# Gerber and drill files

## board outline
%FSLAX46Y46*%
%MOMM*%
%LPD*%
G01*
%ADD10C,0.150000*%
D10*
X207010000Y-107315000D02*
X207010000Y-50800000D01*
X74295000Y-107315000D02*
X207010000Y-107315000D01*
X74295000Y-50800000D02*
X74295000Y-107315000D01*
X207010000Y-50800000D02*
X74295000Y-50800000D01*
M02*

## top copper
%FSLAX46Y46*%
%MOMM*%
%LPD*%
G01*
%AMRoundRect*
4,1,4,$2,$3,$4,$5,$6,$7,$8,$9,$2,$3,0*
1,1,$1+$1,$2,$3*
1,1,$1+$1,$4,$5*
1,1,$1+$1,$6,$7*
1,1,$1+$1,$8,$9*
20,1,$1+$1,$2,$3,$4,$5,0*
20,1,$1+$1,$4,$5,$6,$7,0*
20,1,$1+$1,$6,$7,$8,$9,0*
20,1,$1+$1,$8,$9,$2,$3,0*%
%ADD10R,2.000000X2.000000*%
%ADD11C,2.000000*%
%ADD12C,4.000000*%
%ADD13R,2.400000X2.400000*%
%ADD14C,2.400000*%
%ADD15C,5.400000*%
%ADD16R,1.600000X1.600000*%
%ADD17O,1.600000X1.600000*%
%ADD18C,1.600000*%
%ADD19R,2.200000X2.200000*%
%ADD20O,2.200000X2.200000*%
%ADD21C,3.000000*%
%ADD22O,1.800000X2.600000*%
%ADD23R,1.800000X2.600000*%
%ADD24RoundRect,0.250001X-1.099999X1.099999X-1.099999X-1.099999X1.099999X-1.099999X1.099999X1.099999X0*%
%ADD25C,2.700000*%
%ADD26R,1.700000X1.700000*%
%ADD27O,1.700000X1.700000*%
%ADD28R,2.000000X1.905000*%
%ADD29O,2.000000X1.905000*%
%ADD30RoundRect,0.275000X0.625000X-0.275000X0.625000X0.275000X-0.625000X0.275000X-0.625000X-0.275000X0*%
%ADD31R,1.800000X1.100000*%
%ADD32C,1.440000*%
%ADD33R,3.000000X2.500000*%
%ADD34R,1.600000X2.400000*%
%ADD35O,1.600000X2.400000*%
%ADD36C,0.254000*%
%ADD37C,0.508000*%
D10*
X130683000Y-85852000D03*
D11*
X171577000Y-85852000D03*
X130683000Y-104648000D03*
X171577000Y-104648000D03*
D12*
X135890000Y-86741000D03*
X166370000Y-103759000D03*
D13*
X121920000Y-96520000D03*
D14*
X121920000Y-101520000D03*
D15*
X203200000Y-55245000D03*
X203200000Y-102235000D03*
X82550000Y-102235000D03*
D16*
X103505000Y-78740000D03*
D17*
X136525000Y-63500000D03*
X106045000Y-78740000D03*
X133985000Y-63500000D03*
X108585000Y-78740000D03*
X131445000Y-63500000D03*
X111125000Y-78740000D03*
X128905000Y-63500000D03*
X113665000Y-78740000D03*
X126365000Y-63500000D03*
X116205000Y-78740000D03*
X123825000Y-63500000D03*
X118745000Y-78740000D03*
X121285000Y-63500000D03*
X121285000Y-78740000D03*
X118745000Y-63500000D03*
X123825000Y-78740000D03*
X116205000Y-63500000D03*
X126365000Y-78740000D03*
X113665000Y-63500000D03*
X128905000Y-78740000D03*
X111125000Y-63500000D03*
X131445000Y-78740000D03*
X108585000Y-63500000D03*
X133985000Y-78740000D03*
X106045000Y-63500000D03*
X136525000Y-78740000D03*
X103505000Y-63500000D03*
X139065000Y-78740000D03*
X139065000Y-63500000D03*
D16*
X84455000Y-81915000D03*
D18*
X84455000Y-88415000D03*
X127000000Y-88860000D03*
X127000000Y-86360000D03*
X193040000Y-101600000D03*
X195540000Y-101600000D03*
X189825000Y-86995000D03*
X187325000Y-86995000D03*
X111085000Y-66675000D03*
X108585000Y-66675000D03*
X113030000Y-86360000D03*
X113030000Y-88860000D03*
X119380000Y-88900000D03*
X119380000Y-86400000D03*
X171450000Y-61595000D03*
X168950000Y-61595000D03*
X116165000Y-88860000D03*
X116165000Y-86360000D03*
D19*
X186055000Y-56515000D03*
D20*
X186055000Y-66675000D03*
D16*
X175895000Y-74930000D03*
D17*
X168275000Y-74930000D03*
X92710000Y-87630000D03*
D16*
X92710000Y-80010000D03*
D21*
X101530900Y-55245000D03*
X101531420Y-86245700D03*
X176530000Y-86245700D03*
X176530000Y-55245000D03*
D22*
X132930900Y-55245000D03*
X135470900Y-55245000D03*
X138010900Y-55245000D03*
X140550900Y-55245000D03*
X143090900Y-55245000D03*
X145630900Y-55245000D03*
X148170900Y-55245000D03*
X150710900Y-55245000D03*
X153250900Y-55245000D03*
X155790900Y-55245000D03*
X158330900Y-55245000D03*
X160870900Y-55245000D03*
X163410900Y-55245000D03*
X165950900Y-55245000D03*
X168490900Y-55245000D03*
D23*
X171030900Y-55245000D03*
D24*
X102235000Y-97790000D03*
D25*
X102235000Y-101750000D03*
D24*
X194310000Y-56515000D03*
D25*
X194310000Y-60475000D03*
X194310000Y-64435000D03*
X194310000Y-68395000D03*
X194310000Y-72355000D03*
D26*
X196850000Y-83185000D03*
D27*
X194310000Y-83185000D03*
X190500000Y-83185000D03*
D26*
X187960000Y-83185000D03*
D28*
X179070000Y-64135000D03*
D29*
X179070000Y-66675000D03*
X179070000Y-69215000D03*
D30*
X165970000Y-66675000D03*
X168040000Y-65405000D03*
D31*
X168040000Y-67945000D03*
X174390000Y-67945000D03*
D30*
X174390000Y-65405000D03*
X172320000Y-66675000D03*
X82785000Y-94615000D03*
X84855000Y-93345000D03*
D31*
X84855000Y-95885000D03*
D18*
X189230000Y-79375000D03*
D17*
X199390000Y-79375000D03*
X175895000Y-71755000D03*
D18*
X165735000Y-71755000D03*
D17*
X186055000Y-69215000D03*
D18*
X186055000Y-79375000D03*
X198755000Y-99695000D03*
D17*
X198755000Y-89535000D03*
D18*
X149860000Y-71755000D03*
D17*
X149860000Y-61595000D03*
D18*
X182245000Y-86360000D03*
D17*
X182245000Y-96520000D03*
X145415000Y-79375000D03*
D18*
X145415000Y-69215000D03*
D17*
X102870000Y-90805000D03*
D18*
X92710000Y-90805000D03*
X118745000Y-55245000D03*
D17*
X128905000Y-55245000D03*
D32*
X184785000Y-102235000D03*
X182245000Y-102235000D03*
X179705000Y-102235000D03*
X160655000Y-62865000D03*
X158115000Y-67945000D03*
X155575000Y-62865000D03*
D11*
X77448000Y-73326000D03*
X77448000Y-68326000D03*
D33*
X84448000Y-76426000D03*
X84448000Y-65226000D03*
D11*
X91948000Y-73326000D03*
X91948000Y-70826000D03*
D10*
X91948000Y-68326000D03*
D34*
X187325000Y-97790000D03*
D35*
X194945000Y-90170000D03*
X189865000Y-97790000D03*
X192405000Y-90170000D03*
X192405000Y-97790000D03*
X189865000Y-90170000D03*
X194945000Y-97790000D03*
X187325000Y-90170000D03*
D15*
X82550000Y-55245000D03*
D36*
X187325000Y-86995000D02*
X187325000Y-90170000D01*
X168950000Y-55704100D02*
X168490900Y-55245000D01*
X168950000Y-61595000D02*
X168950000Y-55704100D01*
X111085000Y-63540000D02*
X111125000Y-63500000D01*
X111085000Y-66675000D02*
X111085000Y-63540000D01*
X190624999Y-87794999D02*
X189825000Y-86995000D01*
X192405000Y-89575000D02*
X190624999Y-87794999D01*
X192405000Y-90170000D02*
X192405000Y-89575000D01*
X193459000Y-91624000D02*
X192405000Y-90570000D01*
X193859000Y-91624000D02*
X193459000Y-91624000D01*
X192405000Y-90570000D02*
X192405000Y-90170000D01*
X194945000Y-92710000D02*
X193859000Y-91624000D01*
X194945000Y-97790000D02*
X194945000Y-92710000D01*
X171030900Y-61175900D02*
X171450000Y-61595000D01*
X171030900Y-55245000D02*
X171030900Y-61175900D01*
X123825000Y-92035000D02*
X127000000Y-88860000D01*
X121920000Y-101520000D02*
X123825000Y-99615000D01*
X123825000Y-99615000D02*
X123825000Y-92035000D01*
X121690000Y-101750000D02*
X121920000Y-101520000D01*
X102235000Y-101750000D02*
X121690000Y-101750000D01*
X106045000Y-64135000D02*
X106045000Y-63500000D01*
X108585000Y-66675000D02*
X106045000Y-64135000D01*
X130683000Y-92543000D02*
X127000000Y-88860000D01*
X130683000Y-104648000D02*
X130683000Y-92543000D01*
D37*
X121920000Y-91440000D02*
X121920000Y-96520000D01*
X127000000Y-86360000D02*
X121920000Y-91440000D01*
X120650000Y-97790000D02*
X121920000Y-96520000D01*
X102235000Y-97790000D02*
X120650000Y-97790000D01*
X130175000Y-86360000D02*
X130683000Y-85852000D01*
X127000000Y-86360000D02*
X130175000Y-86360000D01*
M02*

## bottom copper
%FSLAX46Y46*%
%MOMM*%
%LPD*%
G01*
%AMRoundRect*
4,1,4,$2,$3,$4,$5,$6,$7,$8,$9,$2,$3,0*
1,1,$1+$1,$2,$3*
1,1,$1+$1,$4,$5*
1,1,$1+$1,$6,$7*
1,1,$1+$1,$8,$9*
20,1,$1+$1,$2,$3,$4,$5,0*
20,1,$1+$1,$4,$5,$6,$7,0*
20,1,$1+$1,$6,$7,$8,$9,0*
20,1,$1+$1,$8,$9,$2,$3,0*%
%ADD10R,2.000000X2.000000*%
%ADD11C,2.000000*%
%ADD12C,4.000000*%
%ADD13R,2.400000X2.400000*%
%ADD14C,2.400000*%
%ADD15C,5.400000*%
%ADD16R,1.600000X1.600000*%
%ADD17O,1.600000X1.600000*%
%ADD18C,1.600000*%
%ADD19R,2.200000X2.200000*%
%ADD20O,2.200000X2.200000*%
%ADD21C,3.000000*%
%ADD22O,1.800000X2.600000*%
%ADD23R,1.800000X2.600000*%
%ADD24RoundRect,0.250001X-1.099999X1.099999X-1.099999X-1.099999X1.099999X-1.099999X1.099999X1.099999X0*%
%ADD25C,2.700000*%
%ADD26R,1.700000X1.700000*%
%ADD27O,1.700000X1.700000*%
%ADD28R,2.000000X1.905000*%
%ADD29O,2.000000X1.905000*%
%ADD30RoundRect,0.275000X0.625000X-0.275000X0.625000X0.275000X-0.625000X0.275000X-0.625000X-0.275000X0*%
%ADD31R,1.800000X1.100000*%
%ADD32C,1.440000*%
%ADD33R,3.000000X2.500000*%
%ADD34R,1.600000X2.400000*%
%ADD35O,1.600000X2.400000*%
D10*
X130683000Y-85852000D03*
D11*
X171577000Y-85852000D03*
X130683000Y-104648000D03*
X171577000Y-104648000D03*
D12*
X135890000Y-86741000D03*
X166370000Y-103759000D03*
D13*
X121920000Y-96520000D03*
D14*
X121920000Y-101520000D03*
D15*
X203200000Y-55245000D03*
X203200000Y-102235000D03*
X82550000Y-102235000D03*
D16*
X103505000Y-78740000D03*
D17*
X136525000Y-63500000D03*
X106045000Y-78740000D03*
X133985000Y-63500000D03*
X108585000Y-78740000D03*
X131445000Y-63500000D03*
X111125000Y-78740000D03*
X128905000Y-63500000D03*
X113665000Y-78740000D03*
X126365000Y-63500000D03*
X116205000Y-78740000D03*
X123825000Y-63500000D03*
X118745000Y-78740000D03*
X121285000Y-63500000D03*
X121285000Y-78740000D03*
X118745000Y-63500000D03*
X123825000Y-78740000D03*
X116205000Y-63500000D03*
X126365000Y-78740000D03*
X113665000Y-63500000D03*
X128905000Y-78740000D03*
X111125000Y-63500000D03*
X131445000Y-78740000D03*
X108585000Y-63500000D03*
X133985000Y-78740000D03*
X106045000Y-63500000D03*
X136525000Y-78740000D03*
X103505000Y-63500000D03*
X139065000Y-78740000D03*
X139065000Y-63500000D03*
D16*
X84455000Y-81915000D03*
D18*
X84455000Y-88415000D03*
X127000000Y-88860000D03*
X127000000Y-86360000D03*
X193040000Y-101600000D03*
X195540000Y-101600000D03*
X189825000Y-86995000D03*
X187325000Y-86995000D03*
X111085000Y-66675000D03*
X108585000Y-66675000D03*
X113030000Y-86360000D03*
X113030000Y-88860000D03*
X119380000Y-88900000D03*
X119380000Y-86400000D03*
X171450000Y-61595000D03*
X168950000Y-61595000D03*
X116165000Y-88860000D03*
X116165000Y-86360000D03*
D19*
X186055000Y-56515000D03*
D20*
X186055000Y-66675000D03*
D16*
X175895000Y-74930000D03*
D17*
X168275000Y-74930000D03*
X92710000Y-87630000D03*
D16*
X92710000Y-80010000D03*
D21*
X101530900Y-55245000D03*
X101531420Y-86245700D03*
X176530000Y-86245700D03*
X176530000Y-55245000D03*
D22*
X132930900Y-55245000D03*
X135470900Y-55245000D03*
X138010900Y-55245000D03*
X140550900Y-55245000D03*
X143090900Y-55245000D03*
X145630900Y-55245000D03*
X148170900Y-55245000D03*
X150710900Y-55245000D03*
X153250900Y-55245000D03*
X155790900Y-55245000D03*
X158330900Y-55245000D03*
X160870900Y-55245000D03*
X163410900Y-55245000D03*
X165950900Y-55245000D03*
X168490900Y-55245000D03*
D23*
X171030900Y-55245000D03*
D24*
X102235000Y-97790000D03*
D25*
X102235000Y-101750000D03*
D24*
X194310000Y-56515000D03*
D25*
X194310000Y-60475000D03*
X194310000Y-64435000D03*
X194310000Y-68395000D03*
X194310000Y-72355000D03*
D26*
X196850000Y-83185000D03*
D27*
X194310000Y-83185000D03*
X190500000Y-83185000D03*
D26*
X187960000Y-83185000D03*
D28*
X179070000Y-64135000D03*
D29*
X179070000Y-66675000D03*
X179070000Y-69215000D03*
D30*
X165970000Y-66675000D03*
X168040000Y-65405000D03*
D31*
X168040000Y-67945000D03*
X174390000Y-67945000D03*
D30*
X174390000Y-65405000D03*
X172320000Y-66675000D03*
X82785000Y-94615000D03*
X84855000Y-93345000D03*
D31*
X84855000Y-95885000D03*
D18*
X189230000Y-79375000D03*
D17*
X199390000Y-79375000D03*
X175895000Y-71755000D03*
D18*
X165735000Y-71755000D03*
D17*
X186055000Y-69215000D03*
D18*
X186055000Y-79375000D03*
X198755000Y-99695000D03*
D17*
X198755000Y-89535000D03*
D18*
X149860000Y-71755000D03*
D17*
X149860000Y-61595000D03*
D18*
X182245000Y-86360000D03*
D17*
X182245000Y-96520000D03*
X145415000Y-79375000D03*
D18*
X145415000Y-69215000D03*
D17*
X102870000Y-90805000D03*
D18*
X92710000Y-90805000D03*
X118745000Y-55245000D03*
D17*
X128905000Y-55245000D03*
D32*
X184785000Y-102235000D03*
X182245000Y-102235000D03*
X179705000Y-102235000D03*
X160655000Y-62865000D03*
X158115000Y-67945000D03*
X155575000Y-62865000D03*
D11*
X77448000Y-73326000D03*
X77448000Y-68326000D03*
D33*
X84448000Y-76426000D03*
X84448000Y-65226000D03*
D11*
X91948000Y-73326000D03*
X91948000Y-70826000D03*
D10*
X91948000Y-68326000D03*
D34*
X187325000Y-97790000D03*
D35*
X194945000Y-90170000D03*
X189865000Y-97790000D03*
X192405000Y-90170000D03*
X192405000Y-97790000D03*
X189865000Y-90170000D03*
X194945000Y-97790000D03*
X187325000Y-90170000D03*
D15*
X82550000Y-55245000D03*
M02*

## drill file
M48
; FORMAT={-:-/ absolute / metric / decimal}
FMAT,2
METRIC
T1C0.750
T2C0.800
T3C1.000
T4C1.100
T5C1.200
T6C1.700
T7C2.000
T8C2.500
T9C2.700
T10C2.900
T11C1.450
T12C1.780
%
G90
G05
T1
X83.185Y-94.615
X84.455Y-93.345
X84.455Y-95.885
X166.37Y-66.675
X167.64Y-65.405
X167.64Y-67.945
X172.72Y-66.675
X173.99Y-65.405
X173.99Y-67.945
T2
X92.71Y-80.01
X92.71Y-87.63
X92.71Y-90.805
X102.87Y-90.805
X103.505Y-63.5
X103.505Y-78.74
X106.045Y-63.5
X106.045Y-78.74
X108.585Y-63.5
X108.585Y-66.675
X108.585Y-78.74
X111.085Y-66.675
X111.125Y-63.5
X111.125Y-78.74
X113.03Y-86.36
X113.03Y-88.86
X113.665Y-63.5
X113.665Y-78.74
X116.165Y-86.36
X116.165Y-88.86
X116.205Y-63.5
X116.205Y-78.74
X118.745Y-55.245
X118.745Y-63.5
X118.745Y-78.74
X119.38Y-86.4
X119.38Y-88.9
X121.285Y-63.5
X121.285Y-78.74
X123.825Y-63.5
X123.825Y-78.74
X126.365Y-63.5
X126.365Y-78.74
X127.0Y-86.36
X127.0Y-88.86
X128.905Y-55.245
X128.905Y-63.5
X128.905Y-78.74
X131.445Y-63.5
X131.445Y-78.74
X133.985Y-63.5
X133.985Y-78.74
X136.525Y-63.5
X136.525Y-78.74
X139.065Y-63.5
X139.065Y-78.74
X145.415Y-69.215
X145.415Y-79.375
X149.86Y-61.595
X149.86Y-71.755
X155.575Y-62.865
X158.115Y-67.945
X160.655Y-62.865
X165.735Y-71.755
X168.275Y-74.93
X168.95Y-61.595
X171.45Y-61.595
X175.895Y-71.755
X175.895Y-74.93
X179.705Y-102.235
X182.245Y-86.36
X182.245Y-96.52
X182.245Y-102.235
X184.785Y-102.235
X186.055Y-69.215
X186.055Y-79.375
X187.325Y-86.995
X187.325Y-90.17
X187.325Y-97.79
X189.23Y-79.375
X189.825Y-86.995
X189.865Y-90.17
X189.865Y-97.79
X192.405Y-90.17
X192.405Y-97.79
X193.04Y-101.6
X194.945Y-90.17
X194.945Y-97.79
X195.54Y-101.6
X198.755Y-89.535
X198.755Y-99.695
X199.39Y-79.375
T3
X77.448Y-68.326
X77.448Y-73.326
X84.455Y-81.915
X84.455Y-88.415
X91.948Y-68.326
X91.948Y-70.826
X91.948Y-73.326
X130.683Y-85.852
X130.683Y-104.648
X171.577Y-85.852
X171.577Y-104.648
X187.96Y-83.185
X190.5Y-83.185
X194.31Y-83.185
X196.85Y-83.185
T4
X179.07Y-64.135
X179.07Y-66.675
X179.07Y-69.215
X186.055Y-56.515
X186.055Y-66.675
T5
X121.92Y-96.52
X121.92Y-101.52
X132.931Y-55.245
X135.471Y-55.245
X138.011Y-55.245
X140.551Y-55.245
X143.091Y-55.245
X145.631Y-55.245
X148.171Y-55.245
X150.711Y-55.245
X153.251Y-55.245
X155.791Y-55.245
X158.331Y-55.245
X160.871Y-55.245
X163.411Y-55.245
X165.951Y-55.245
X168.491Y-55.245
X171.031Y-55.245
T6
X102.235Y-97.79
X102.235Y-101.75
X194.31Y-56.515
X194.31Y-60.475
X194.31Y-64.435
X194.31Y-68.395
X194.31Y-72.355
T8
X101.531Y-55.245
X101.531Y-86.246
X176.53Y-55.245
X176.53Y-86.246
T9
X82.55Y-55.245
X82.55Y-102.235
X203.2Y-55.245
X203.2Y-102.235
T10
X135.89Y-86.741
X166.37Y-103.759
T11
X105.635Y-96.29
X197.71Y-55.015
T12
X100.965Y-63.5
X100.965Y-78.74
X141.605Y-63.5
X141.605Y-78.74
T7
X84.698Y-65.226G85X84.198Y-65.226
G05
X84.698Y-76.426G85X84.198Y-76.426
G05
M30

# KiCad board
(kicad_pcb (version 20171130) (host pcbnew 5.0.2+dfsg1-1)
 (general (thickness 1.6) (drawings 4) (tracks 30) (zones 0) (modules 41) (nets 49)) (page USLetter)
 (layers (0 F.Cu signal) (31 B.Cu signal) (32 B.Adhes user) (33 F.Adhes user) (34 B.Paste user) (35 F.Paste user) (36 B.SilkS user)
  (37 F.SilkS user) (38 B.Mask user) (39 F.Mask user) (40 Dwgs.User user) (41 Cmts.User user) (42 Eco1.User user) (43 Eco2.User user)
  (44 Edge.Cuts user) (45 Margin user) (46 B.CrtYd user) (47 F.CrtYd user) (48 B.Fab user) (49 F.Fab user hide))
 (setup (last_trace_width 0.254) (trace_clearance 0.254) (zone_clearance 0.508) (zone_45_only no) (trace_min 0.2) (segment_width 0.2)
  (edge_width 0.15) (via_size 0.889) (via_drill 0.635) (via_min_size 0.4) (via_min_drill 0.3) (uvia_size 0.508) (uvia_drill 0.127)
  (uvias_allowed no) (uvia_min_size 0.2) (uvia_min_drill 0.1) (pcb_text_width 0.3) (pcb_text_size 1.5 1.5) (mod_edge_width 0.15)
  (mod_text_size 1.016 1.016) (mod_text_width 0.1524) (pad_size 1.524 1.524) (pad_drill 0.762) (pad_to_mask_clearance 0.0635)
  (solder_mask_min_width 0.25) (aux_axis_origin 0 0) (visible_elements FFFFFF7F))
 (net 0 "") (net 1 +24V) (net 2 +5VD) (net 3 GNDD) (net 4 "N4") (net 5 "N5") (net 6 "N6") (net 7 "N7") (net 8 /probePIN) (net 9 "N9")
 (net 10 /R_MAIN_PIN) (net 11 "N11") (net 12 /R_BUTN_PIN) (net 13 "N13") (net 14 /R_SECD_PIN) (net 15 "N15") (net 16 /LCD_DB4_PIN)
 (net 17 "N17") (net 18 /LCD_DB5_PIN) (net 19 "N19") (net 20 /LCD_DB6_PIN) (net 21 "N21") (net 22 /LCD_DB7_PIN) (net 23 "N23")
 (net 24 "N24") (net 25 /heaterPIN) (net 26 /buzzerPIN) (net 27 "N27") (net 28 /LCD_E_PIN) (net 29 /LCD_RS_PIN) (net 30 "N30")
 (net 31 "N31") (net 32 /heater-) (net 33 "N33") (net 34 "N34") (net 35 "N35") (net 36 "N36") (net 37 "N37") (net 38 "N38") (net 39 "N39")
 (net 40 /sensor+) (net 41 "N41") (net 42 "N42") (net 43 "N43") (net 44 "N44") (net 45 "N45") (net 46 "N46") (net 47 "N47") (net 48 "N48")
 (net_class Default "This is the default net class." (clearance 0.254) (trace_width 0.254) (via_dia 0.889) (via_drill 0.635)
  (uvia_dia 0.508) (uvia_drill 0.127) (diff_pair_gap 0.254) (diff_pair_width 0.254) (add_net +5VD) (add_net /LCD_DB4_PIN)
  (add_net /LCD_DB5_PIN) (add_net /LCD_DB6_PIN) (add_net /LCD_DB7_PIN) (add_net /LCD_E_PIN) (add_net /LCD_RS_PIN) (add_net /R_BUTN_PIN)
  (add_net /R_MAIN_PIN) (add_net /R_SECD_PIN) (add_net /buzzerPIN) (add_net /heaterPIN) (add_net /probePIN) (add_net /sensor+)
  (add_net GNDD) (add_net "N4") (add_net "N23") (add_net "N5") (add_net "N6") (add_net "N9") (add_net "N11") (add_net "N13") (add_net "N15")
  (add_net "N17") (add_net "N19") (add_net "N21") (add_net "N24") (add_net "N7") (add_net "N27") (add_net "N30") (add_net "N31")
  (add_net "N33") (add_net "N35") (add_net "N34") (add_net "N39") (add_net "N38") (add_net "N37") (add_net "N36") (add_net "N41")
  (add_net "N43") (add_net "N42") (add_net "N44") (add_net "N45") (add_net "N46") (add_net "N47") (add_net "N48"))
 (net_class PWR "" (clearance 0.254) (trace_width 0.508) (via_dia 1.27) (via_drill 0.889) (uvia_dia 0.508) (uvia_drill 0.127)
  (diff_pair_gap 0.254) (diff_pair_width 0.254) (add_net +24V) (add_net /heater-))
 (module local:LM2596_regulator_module (layer F.Cu) (at 151.13 95.25)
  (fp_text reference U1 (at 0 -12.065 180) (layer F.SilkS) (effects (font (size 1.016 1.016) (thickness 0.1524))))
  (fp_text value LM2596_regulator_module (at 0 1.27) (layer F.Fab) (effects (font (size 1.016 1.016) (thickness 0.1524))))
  (pad 1 thru_hole rect (at -20.447 -9.398) (size 2 2) (drill 1) (layers *.Cu *.Mask) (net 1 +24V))
  (pad 4 thru_hole circle (at 20.447 -9.398) (size 2 2) (drill 1) (layers *.Cu *.Mask) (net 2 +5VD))
  (pad 2 thru_hole circle (at -20.447 9.398) (size 2 2) (drill 1) (layers *.Cu *.Mask) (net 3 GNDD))
  (pad 3 thru_hole circle (at 20.447 9.398) (size 2 2) (drill 1) (layers *.Cu *.Mask) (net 3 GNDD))
  (pad "" thru_hole circle (at -15.24 -8.509) (size 4 4) (drill 2.9) (layers *.Cu *.Mask))
  (pad "" thru_hole circle (at 15.24 8.509) (size 4 4) (drill 2.9) (layers *.Cu *.Mask)))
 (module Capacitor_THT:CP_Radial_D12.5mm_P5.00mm (layer F.Cu) (at 121.92 96.52 270)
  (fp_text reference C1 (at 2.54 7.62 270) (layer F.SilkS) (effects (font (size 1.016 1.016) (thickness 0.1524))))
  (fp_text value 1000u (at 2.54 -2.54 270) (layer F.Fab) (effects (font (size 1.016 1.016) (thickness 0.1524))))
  (pad 1 thru_hole rect (at 0 0 270) (size 2.4 2.4) (drill 1.2) (layers *.Cu *.Mask) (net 1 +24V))
  (pad 2 thru_hole circle (at 5 0 270) (size 2.4 2.4) (drill 1.2) (layers *.Cu *.Mask) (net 3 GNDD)))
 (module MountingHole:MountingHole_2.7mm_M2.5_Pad (layer F.Cu) (at 203.2 55.245)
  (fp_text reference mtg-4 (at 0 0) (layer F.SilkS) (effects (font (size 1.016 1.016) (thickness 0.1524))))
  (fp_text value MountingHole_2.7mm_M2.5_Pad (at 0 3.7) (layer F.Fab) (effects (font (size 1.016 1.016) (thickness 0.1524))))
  (pad 1 thru_hole circle (at 0 0) (size 5.4 5.4) (drill 2.7) (layers *.Cu *.Mask)))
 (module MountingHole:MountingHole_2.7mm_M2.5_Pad (layer F.Cu) (at 203.2 102.235)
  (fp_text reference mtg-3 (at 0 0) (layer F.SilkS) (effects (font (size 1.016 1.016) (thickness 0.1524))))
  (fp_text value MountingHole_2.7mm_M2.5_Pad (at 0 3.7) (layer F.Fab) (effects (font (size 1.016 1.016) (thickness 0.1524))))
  (pad 1 thru_hole circle (at 0 0) (size 5.4 5.4) (drill 2.7) (layers *.Cu *.Mask)))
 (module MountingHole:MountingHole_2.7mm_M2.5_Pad (layer F.Cu) (at 82.55 102.235)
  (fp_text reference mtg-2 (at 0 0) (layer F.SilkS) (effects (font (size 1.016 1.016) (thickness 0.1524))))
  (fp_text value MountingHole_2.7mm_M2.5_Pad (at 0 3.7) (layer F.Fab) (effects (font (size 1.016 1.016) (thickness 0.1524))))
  (pad 1 thru_hole circle (at 0 0) (size 5.4 5.4) (drill 2.7) (layers *.Cu *.Mask)))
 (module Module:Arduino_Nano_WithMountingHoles (layer F.Cu) (at 103.505 78.74 90)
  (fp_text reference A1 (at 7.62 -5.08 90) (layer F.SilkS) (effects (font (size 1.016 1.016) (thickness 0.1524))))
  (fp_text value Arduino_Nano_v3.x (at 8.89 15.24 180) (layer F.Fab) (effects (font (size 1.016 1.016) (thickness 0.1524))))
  (pad 1 thru_hole rect (at 0 0 90) (size 1.6 1.6) (drill 0.8) (layers *.Cu *.Mask) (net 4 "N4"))
  (pad 17 thru_hole oval (at 15.24 33.02 90) (size 1.6 1.6) (drill 0.8) (layers *.Cu *.Mask) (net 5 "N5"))
  (pad 2 thru_hole oval (at 0 2.54 90) (size 1.6 1.6) (drill 0.8) (layers *.Cu *.Mask) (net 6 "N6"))
  (pad 18 thru_hole oval (at 15.24 30.48 90) (size 1.6 1.6) (drill 0.8) (layers *.Cu *.Mask) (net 2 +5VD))
  (pad 3 thru_hole oval (at 0 5.08 90) (size 1.6 1.6) (drill 0.8) (layers *.Cu *.Mask) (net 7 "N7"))
  (pad 19 thru_hole oval (at 15.24 27.94 90) (size 1.6 1.6) (drill 0.8) (layers *.Cu *.Mask) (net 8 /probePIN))
  (pad 4 thru_hole oval (at 0 7.62 90) (size 1.6 1.6) (drill 0.8) (layers *.Cu *.Mask) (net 3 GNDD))
  (pad 20 thru_hole oval (at 15.24 25.4 90) (size 1.6 1.6) (drill 0.8) (layers *.Cu *.Mask) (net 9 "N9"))
  (pad 5 thru_hole oval (at 0 10.16 90) (size 1.6 1.6) (drill 0.8) (layers *.Cu *.Mask) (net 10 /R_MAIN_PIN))
  (pad 21 thru_hole oval (at 15.24 22.86 90) (size 1.6 1.6) (drill 0.8) (layers *.Cu *.Mask) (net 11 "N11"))
  (pad 6 thru_hole oval (at 0 12.7 90) (size 1.6 1.6) (drill 0.8) (layers *.Cu *.Mask) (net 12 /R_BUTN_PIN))
  (pad 22 thru_hole oval (at 15.24 20.32 90) (size 1.6 1.6) (drill 0.8) (layers *.Cu *.Mask) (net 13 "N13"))
  (pad 7 thru_hole oval (at 0 15.24 90) (size 1.6 1.6) (drill 0.8) (layers *.Cu *.Mask) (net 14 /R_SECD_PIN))
  (pad 23 thru_hole oval (at 15.24 17.78 90) (size 1.6 1.6) (drill 0.8) (layers *.Cu *.Mask) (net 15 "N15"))
  (pad 8 thru_hole oval (at 0 17.78 90) (size 1.6 1.6) (drill 0.8) (layers *.Cu *.Mask) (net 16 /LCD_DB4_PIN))
  (pad 24 thru_hole oval (at 15.24 15.24 90) (size 1.6 1.6) (drill 0.8) (layers *.Cu *.Mask) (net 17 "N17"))
  (pad 9 thru_hole oval (at 0 20.32 90) (size 1.6 1.6) (drill 0.8) (layers *.Cu *.Mask) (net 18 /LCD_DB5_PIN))
  (pad 25 thru_hole oval (at 15.24 12.7 90) (size 1.6 1.6) (drill 0.8) (layers *.Cu *.Mask) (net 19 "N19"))
  (pad 10 thru_hole oval (at 0 22.86 90) (size 1.6 1.6) (drill 0.8) (layers *.Cu *.Mask) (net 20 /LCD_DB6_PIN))
  (pad 26 thru_hole oval (at 15.24 10.16 90) (size 1.6 1.6) (drill 0.8) (layers *.Cu *.Mask) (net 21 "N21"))
  (pad 11 thru_hole oval (at 0 25.4 90) (size 1.6 1.6) (drill 0.8) (layers *.Cu *.Mask) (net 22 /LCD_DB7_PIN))
  (pad 27 thru_hole oval (at 15.24 7.62 90) (size 1.6 1.6) (drill 0.8) (layers *.Cu *.Mask) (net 2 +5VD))
  (pad 12 thru_hole oval (at 0 27.94 90) (size 1.6 1.6) (drill 0.8) (layers *.Cu *.Mask) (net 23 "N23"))
  (pad 28 thru_hole oval (at 15.24 5.08 90) (size 1.6 1.6) (drill 0.8) (layers *.Cu *.Mask) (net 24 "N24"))
  (pad 13 thru_hole oval (at 0 30.48 90) (size 1.6 1.6) (drill 0.8) (layers *.Cu *.Mask) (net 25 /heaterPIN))
  (pad 29 thru_hole oval (at 15.24 2.54 90) (size 1.6 1.6) (drill 0.8) (layers *.Cu *.Mask) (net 3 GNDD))
  (pad 14 thru_hole oval (at 0 33.02 90) (size 1.6 1.6) (drill 0.8) (layers *.Cu *.Mask) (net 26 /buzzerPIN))
  (pad 30 thru_hole oval (at 15.24 0 90) (size 1.6 1.6) (drill 0.8) (layers *.Cu *.Mask) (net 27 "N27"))
  (pad 15 thru_hole oval (at 0 35.56 90) (size 1.6 1.6) (drill 0.8) (layers *.Cu *.Mask) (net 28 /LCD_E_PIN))
  (pad 16 thru_hole oval (at 15.24 35.56 90) (size 1.6 1.6) (drill 0.8) (layers *.Cu *.Mask) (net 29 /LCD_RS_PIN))
  (pad "" np_thru_hole circle (at 0 -2.54 90) (size 1.78 1.78) (drill 1.78) (layers *.Cu *.Mask))
  (pad "" np_thru_hole circle (at 15.24 -2.54 90) (size 1.78 1.78) (drill 1.78) (layers *.Cu *.Mask))
  (pad "" np_thru_hole circle (at 15.24 38.1 90) (size 1.78 1.78) (drill 1.78) (layers *.Cu *.Mask))
  (pad "" np_thru_hole circle (at 0 38.1 90) (size 1.78 1.78) (drill 1.78) (layers *.Cu *.Mask)))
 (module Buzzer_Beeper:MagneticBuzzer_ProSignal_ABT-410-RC (layer F.Cu) (at 84.455 81.915 270)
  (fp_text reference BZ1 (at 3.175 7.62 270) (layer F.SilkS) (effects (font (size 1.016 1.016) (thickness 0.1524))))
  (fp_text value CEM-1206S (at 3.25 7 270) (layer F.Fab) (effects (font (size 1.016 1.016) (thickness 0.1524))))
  (pad 1 thru_hole rect (at 0 0 270) (size 1.6 1.6) (drill 1) (layers *.Cu *.Mask) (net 2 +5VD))
  (pad 2 thru_hole circle (at 6.5 0 270) (size 1.6 1.6) (drill 1) (layers *.Cu *.Mask) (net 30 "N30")))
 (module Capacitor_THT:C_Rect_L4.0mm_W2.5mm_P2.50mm (layer F.Cu) (at 127 86.36 270)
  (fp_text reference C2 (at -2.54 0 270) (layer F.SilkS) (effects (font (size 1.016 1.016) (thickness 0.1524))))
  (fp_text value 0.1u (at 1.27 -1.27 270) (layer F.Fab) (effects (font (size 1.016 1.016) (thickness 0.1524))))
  (pad 2 thru_hole circle (at 2.5 0 270) (size 1.6 1.6) (drill 0.8) (layers *.Cu *.Mask) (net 3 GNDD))
  (pad 1 thru_hole circle (at 0 0 270) (size 1.6 1.6) (drill 0.8) (layers *.Cu *.Mask) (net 1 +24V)))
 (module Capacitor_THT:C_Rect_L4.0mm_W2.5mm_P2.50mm (layer F.Cu) (at 193.04 101.6)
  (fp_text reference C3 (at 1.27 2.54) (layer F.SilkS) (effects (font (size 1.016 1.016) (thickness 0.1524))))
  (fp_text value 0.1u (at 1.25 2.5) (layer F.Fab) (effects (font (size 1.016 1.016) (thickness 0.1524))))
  (pad 1 thru_hole circle (at 0 0) (size 1.6 1.6) (drill 0.8) (layers *.Cu *.Mask) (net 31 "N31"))
  (pad 2 thru_hole circle (at 2.5 0) (size 1.6 1.6) (drill 0.8) (layers *.Cu *.Mask) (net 3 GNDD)))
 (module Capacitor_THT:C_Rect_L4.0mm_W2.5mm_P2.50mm (layer F.Cu) (at 187.325 86.995)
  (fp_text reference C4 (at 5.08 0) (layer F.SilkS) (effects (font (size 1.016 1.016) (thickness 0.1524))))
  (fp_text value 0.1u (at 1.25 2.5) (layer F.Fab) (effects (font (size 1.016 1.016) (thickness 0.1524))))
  (pad 2 thru_hole circle (at 2.5 0) (size 1.6 1.6) (drill 0.8) (layers *.Cu *.Mask) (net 3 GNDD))
  (pad 1 thru_hole circle (at 0 0) (size 1.6 1.6) (drill 0.8) (layers *.Cu *.Mask) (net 2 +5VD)))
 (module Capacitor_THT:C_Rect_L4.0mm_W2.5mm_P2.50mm (layer F.Cu) (at 108.585 66.675)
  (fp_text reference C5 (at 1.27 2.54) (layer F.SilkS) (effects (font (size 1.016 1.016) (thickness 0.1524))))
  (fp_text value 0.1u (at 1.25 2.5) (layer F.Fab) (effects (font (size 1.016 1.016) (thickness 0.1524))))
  (pad 2 thru_hole circle (at 2.5 0) (size 1.6 1.6) (drill 0.8) (layers *.Cu *.Mask) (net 2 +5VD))
  (pad 1 thru_hole circle (at 0 0) (size 1.6 1.6) (drill 0.8) (layers *.Cu *.Mask) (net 3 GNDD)))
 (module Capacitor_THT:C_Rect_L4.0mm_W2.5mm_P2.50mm (layer F.Cu) (at 113.03 86.36 270)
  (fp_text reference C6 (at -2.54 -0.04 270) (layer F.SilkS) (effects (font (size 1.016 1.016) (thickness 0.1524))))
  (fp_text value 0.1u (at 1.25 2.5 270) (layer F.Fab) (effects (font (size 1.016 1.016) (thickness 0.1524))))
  (pad 1 thru_hole circle (at 0 0 270) (size 1.6 1.6) (drill 0.8) (layers *.Cu *.Mask) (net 10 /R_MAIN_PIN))
  (pad 2 thru_hole circle (at 2.5 0 270) (size 1.6 1.6) (drill 0.8) (layers *.Cu *.Mask) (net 3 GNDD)))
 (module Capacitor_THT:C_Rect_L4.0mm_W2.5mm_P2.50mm (layer F.Cu) (at 119.38 88.9 90)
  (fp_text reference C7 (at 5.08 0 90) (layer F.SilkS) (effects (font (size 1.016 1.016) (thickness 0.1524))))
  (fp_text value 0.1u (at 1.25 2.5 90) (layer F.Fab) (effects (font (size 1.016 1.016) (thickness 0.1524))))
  (pad 1 thru_hole circle (at 0 0 90) (size 1.6 1.6) (drill 0.8) (layers *.Cu *.Mask) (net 3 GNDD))
  (pad 2 thru_hole circle (at 2.5 0 90) (size 1.6 1.6) (drill 0.8) (layers *.Cu *.Mask) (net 14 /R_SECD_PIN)))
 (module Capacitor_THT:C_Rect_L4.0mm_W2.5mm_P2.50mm (layer F.Cu) (at 171.45 61.595 180)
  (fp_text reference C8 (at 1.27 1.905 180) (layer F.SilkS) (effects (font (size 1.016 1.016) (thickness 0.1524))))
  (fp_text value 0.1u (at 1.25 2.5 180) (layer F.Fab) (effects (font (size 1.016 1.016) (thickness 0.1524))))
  (pad 1 thru_hole circle (at 0 0 180) (size 1.6 1.6) (drill 0.8) (layers *.Cu *.Mask) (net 3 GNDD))
  (pad 2 thru_hole circle (at 2.5 0 180) (size 1.6 1.6) (drill 0.8) (layers *.Cu *.Mask) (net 2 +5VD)))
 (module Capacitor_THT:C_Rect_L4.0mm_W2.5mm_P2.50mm (layer F.Cu) (at 116.165 86.36 270)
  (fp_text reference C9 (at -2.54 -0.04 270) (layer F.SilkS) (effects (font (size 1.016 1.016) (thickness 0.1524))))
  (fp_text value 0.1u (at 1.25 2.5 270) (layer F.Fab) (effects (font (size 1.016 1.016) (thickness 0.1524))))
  (pad 2 thru_hole circle (at 2.5 0 270) (size 1.6 1.6) (drill 0.8) (layers *.Cu *.Mask) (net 3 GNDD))
  (pad 1 thru_hole circle (at 0 0 270) (size 1.6 1.6) (drill 0.8) (layers *.Cu *.Mask) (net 12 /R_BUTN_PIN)))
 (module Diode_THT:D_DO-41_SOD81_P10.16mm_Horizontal (layer F.Cu) (at 186.055 56.515 270)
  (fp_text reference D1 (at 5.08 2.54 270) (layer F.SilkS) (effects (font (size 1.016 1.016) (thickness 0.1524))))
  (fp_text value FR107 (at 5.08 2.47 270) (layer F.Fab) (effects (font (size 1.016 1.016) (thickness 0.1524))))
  (pad 1 thru_hole rect (at 0 0 270) (size 2.2 2.2) (drill 1.1) (layers *.Cu *.Mask) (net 1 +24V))
  (pad 2 thru_hole oval (at 10.16 0 270) (size 2.2 2.2) (drill 1.1) (layers *.Cu *.Mask) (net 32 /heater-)))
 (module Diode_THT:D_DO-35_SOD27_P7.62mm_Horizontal (layer F.Cu) (at 175.895 74.93 180)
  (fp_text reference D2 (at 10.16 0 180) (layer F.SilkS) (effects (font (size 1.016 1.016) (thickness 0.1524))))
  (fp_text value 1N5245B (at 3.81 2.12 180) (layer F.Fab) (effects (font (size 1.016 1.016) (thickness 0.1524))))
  (pad 1 thru_hole rect (at 0 0 180) (size 1.6 1.6) (drill 0.8) (layers *.Cu *.Mask) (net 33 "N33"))
  (pad 2 thru_hole oval (at 7.62 0 180) (size 1.6 1.6) (drill 0.8) (layers *.Cu *.Mask) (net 3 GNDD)))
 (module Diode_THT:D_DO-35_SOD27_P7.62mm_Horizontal (layer F.Cu) (at 92.71 80.01 270)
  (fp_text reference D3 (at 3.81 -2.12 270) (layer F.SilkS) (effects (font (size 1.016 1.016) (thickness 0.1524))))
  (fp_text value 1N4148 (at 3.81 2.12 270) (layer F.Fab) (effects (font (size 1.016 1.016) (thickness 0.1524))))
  (pad 2 thru_hole oval (at 7.62 0 270) (size 1.6 1.6) (drill 0.8) (layers *.Cu *.Mask) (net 30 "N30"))
  (pad 1 thru_hole rect (at 0 0 270) (size 1.6 1.6) (drill 0.8) (layers *.Cu *.Mask) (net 2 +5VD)))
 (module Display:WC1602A (layer B.Cu) (at 171.0309 55.245 180)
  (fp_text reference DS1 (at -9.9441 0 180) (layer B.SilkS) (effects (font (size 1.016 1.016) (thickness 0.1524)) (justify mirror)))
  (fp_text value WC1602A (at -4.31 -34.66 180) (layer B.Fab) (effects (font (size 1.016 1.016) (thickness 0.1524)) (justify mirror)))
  (pad "" thru_hole circle (at 69.5 0 180) (size 3 3) (drill 2.5) (layers *.Cu *.Mask))
  (pad "" thru_hole circle (at 69.49948 -31.0007 180) (size 3 3) (drill 2.5) (layers *.Cu *.Mask))
  (pad "" thru_hole circle (at -5.4991 -31.0007 180) (size 3 3) (drill 2.5) (layers *.Cu *.Mask))
  (pad "" thru_hole circle (at -5.4991 0 180) (size 3 3) (drill 2.5) (layers *.Cu *.Mask))
  (pad 16 thru_hole oval (at 38.1 0 180) (size 1.8 2.6) (drill 1.2) (layers *.Cu *.Mask) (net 3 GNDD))
  (pad 15 thru_hole oval (at 35.56 0 180) (size 1.8 2.6) (drill 1.2) (layers *.Cu *.Mask) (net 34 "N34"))
  (pad 14 thru_hole oval (at 33.02 0 180) (size 1.8 2.6) (drill 1.2) (layers *.Cu *.Mask) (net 22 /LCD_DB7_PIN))
  (pad 13 thru_hole oval (at 30.48 0 180) (size 1.8 2.6) (drill 1.2) (layers *.Cu *.Mask) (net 20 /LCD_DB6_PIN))
  (pad 12 thru_hole oval (at 27.94 0 180) (size 1.8 2.6) (drill 1.2) (layers *.Cu *.Mask) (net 18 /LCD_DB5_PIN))
  (pad 11 thru_hole oval (at 25.4 0 180) (size 1.8 2.6) (drill 1.2) (layers *.Cu *.Mask) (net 16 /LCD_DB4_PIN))
  (pad 10 thru_hole oval (at 22.86 0 180) (size 1.8 2.6) (drill 1.2) (layers *.Cu *.Mask) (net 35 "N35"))
  (pad 9 thru_hole oval (at 20.32 0 180) (size 1.8 2.6) (drill 1.2) (layers *.Cu *.Mask) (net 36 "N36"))
  (pad 8 thru_hole oval (at 17.78 0 180) (size 1.8 2.6) (drill 1.2) (layers *.Cu *.Mask) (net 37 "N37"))
  (pad 7 thru_hole oval (at 15.24 0 180) (size 1.8 2.6) (drill 1.2) (layers *.Cu *.Mask) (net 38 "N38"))
  (pad 6 thru_hole oval (at 12.7 0 180) (size 1.8 2.6) (drill 1.2) (layers *.Cu *.Mask) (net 28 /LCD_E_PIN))
  (pad 5 thru_hole oval (at 10.16 0 180) (size 1.8 2.6) (drill 1.2) (layers *.Cu *.Mask) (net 3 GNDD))
  (pad 4 thru_hole oval (at 7.62 0 180) (size 1.8 2.6) (drill 1.2) (layers *.Cu *.Mask) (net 29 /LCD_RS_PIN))
  (pad 3 thru_hole oval (at 5.08 0 180) (size 1.8 2.6) (drill 1.2) (layers *.Cu *.Mask) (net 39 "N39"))
  (pad 2 thru_hole oval (at 2.54 0 180) (size 1.8 2.6) (drill 1.2) (layers *.Cu *.Mask) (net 2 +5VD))
  (pad 1 thru_hole rect (at 0 0 180) (size 1.8 2.6) (drill 1.2) (layers *.Cu *.Mask) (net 3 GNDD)))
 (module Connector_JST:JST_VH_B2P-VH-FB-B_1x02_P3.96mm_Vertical (layer F.Cu) (at 102.235 97.79 270)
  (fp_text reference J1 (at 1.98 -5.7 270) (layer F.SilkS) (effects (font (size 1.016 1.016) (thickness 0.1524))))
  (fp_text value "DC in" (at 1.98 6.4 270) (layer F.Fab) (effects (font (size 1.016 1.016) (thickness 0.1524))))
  (pad 1 thru_hole roundrect (at 0 0 270) (size 2.7 2.7) (drill 1.7) (layers *.Cu *.Mask) (roundrect_rratio 0.09259299999999999)
   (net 1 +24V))
  (pad 2 thru_hole circle (at 3.96 0 270) (size 2.7 2.7) (drill 1.7) (layers *.Cu *.Mask) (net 3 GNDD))
  (pad "" np_thru_hole circle (at -1.5 -3.4 270) (size 1.45 1.45) (drill 1.45) (layers *.Cu *.Mask)))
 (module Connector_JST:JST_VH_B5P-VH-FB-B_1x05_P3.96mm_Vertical (layer F.Cu) (at 194.31 56.515 270)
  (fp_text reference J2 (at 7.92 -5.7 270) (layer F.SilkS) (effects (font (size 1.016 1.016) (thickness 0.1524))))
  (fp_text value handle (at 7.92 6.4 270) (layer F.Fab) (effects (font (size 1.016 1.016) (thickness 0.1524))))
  (pad 1 thru_hole roundrect (at 0 0 270) (size 2.7 2.7) (drill 1.7) (layers *.Cu *.Mask) (roundrect_rratio 0.09259299999999999)
   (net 1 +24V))
  (pad 2 thru_hole circle (at 3.96 0 270) (size 2.7 2.7) (drill 1.7) (layers *.Cu *.Mask) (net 32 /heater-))
  (pad 3 thru_hole circle (at 7.92 0 270) (size 2.7 2.7) (drill 1.7) (layers *.Cu *.Mask) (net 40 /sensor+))
  (pad 4 thru_hole circle (at 11.88 0 270) (size 2.7 2.7) (drill 1.7) (layers *.Cu *.Mask) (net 3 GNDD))
  (pad 5 thru_hole circle (at 15.84 0 270) (size 2.7 2.7) (drill 1.7) (layers *.Cu *.Mask) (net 3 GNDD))
  (pad "" np_thru_hole circle (at -1.5 -3.4 270) (size 1.45 1.45) (drill 1.45) (layers *.Cu *.Mask)))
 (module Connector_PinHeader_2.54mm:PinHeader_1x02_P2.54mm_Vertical (layer F.Cu) (at 196.85 83.185 270)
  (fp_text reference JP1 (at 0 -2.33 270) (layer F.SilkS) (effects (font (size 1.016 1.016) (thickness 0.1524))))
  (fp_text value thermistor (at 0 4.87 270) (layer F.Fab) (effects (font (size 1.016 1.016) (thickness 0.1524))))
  (pad 1 thru_hole rect (at 0 0 270) (size 1.7 1.7) (drill 1) (layers *.Cu *.Mask) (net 40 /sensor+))
  (pad 2 thru_hole oval (at 0 2.54 270) (size 1.7 1.7) (drill 1) (layers *.Cu *.Mask) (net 31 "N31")))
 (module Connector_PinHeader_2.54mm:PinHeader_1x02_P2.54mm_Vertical (layer F.Cu) (at 187.96 83.185 90)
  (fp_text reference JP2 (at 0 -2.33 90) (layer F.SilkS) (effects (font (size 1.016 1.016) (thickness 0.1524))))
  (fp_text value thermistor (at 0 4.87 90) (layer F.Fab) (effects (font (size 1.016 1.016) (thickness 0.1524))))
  (pad 2 thru_hole oval (at 0 2.54 90) (size 1.7 1.7) (drill 1) (layers *.Cu *.Mask) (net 31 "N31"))
  (pad 1 thru_hole rect (at 0 0 90) (size 1.7 1.7) (drill 1) (layers *.Cu *.Mask) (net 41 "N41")))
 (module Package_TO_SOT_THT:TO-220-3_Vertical (layer F.Cu) (at 179.07 64.135 270)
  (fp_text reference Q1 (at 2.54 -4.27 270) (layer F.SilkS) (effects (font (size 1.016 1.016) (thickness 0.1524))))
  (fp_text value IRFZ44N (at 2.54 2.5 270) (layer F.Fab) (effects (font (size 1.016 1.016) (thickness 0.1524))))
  (pad 1 thru_hole rect (at 0 0 270) (size 1.905 2) (drill 1.1) (layers *.Cu *.Mask) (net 33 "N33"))
  (pad 2 thru_hole oval (at 2.54 0 270) (size 1.905 2) (drill 1.1) (layers *.Cu *.Mask) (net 32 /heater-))
  (pad 3 thru_hole oval (at 5.08 0 270) (size 1.905 2) (drill 1.1) (layers *.Cu *.Mask) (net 3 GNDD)))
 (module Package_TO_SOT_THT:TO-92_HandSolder (layer F.Cu) (at 167.64 67.945 90)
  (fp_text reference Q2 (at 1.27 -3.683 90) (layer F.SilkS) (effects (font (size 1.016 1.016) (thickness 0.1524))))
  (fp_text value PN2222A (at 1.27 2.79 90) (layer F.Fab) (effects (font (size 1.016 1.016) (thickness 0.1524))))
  (pad 2 thru_hole roundrect (at 1.27 -1.27 90) (size 1.1 1.8) (drill 0.75 (offset 0 -0.4)) (layers *.Cu *.Mask) (roundrect_rratio 0.25)
   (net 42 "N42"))
  (pad 3 thru_hole roundrect (at 2.54 0 90) (size 1.1 1.8) (drill 0.75 (offset 0 0.4)) (layers *.Cu *.Mask) (roundrect_rratio 0.25)
   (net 1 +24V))
  (pad 1 thru_hole rect (at 0 0 90) (size 1.1 1.8) (drill 0.75 (offset 0 0.4)) (layers *.Cu *.Mask) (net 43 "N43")))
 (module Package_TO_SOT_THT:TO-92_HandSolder (layer F.Cu) (at 173.99 67.945 90)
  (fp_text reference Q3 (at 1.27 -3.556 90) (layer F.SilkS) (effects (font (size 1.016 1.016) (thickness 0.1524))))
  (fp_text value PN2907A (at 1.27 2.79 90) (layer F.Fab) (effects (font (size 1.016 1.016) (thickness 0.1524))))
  (pad 1 thru_hole rect (at 0 0 90) (size 1.1 1.8) (drill 0.75 (offset 0 0.4)) (layers *.Cu *.Mask) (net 43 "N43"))
  (pad 3 thru_hole roundrect (at 2.54 0 90) (size 1.1 1.8) (drill 0.75 (offset 0 0.4)) (layers *.Cu *.Mask) (roundrect_rratio 0.25)
   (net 3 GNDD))
  (pad 2 thru_hole roundrect (at 1.27 -1.27 90) (size 1.1 1.8) (drill 0.75 (offset 0 -0.4)) (layers *.Cu *.Mask) (roundrect_rratio 0.25)
   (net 42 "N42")))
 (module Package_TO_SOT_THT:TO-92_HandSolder (layer F.Cu) (at 84.455 95.885 90)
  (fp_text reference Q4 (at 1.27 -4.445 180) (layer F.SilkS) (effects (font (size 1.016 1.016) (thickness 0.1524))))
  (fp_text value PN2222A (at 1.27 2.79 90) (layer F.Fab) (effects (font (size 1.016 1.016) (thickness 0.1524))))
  (pad 2 thru_hole roundrect (at 1.27 -1.27 90) (size 1.1 1.8) (drill 0.75 (offset 0 -0.4)) (layers *.Cu *.Mask) (roundrect_rratio 0.25)
   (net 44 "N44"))
  (pad 3 thru_hole roundrect (at 2.54 0 90) (size 1.1 1.8) (drill 0.75 (offset 0 0.4)) (layers *.Cu *.Mask) (roundrect_rratio 0.25)
   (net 30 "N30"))
  (pad 1 thru_hole rect (at 0 0 90) (size 1.1 1.8) (drill 0.75 (offset 0 0.4)) (layers *.Cu *.Mask) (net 3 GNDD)))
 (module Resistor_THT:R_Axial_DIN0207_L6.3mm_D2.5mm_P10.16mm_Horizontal (layer F.Cu) (at 189.23 79.375)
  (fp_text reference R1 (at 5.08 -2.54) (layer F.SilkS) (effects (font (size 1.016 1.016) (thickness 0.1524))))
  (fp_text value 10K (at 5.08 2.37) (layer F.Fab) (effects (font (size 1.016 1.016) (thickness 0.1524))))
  (pad 1 thru_hole circle (at 0 0) (size 1.6 1.6) (drill 0.8) (layers *.Cu *.Mask) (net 31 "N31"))
  (pad 2 thru_hole oval (at 10.16 0) (size 1.6 1.6) (drill 0.8) (layers *.Cu *.Mask) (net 40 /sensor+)))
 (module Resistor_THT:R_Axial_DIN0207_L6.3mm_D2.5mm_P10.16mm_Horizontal (layer F.Cu) (at 165.735 71.755)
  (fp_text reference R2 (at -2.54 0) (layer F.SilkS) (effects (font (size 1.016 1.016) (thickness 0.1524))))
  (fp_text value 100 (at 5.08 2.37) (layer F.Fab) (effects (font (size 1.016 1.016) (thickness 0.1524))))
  (pad 2 thru_hole oval (at 10.16 0) (size 1.6 1.6) (drill 0.8) (layers *.Cu *.Mask) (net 33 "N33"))
  (pad 1 thru_hole circle (at 0 0) (size 1.6 1.6) (drill 0.8) (layers *.Cu *.Mask) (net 43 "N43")))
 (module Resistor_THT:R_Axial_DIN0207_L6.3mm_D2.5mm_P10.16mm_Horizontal (layer F.Cu) (at 186.055 79.375 90)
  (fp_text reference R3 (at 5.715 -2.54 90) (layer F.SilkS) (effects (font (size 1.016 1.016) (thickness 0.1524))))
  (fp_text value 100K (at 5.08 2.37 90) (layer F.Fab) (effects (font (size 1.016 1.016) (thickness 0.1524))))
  (pad 2 thru_hole oval (at 10.16 0 90) (size 1.6 1.6) (drill 0.8) (layers *.Cu *.Mask) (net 2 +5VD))
  (pad 1 thru_hole circle (at 0 0 90) (size 1.6 1.6) (drill 0.8) (layers *.Cu *.Mask) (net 41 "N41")))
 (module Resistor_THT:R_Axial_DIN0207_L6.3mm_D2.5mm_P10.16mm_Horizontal (layer F.Cu) (at 198.755 99.695 90)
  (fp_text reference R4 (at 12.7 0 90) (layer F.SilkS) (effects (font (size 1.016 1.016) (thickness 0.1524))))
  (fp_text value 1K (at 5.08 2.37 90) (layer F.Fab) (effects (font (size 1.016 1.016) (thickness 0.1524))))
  (pad 1 thru_hole circle (at 0 0 90) (size 1.6 1.6) (drill 0.8) (layers *.Cu *.Mask) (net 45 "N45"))
  (pad 2 thru_hole oval (at 10.16 0 90) (size 1.6 1.6) (drill 0.8) (layers *.Cu *.Mask) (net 3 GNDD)))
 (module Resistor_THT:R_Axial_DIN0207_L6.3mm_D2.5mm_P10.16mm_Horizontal (layer F.Cu) (at 149.86 71.755 90)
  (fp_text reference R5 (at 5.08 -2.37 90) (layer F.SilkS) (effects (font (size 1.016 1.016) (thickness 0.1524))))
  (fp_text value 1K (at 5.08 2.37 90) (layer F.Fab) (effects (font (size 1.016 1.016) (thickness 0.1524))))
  (pad 1 thru_hole circle (at 0 0 90) (size 1.6 1.6) (drill 0.8) (layers *.Cu *.Mask) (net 25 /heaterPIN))
  (pad 2 thru_hole oval (at 10.16 0 90) (size 1.6 1.6) (drill 0.8) (layers *.Cu *.Mask) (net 42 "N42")))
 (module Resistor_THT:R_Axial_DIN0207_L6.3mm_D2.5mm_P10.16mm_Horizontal (layer F.Cu) (at 182.245 86.36 270)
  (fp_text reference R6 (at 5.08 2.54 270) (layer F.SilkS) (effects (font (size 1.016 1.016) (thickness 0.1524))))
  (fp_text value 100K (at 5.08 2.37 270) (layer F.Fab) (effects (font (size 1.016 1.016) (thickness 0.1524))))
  (pad 1 thru_hole circle (at 0 0 270) (size 1.6 1.6) (drill 0.8) (layers *.Cu *.Mask) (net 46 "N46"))
  (pad 2 thru_hole oval (at 10.16 0 270) (size 1.6 1.6) (drill 0.8) (layers *.Cu *.Mask) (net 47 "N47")))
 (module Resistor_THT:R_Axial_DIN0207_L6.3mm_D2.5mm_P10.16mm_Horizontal (layer F.Cu) (at 145.415 69.215 270)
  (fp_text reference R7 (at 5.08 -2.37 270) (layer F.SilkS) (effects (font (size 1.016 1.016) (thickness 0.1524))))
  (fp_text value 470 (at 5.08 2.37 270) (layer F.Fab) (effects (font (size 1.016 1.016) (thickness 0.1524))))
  (pad 2 thru_hole oval (at 10.16 0 270) (size 1.6 1.6) (drill 0.8) (layers *.Cu *.Mask) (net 46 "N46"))
  (pad 1 thru_hole circle (at 0 0 270) (size 1.6 1.6) (drill 0.8) (layers *.Cu *.Mask) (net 8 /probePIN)))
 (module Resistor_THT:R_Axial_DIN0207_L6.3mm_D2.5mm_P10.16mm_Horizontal (layer F.Cu) (at 92.71 90.805)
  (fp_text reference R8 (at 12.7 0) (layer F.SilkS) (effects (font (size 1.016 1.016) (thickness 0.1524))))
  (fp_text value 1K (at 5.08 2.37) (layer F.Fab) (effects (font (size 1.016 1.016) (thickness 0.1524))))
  (pad 2 thru_hole oval (at 10.16 0) (size 1.6 1.6) (drill 0.8) (layers *.Cu *.Mask) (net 26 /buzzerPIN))
  (pad 1 thru_hole circle (at 0 0) (size 1.6 1.6) (drill 0.8) (layers *.Cu *.Mask) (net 44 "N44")))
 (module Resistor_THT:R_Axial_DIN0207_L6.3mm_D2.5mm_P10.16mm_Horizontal (layer F.Cu) (at 118.745 55.245)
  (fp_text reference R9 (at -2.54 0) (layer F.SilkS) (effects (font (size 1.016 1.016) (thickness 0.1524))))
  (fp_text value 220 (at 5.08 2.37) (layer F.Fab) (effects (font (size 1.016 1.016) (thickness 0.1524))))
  (pad 1 thru_hole circle (at 0 0) (size 1.6 1.6) (drill 0.8) (layers *.Cu *.Mask) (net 2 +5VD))
  (pad 2 thru_hole oval (at 10.16 0) (size 1.6 1.6) (drill 0.8) (layers *.Cu *.Mask) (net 34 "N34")))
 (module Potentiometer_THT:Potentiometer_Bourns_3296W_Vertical (layer B.Cu) (at 184.785 102.235)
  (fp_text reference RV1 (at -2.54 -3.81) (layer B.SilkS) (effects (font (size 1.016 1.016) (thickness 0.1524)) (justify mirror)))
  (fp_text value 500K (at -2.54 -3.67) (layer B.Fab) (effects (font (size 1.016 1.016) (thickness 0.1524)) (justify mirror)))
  (pad 1 thru_hole circle (at 0 0) (size 1.44 1.44) (drill 0.8) (layers *.Cu *.Mask) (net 45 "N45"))
  (pad 2 thru_hole circle (at -2.54 0) (size 1.44 1.44) (drill 0.8) (layers *.Cu *.Mask) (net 47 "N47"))
  (pad 3 thru_hole circle (at -5.08 0) (size 1.44 1.44) (drill 0.8) (layers *.Cu *.Mask) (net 47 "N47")))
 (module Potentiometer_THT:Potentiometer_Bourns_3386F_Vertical (layer F.Cu) (at 155.575 62.865 270)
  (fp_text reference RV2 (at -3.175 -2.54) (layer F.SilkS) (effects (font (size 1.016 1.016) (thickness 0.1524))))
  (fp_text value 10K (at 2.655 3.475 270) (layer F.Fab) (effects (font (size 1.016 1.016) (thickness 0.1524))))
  (pad 3 thru_hole circle (at 0 -5.08 270) (size 1.44 1.44) (drill 0.8) (layers *.Cu *.Mask) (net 2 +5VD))
  (pad 2 thru_hole circle (at 5.08 -2.54 270) (size 1.44 1.44) (drill 0.8) (layers *.Cu *.Mask) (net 39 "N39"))
  (pad 1 thru_hole circle (at 0 0 270) (size 1.44 1.44) (drill 0.8) (layers *.Cu *.Mask) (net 3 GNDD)))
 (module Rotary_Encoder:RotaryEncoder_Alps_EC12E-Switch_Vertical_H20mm (layer B.Cu) (at 91.948 68.326 180)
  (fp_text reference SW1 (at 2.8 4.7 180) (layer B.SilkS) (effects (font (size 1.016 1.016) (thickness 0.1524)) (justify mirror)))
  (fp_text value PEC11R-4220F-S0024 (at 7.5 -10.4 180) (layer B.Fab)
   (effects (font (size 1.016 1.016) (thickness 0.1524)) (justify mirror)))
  (pad S2 thru_hole circle (at 14.5 -5 180) (size 2 2) (drill 1) (layers *.Cu *.Mask) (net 3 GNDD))
  (pad S1 thru_hole circle (at 14.5 0 180) (size 2 2) (drill 1) (layers *.Cu *.Mask) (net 12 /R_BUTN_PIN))
  (pad MP thru_hole rect (at 7.5 -8.1 180) (size 3 2.5) (drill oval 2.5 2) (layers *.Cu *.Mask))
  (pad MP thru_hole rect (at 7.5 3.1 180) (size 3 2.5) (drill oval 2.5 2) (layers *.Cu *.Mask))
  (pad B thru_hole circle (at 0 -5 180) (size 2 2) (drill 1) (layers *.Cu *.Mask) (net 14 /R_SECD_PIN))
  (pad C thru_hole circle (at 0 -2.5 180) (size 2 2) (drill 1) (layers *.Cu *.Mask) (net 3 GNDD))
  (pad A thru_hole rect (at 0 0 180) (size 2 2) (drill 1) (layers *.Cu *.Mask) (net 10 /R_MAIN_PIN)))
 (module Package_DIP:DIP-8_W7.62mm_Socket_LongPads (layer F.Cu) (at 187.325 97.79 90)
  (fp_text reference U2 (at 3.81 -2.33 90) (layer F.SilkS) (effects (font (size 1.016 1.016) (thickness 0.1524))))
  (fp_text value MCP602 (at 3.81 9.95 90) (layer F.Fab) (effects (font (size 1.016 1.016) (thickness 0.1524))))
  (pad 1 thru_hole rect (at 0 0 90) (size 2.4 1.6) (drill 0.8) (layers *.Cu *.Mask) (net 46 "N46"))
  (pad 5 thru_hole oval (at 7.62 7.62 90) (size 2.4 1.6) (drill 0.8) (layers *.Cu *.Mask) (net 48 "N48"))
  (pad 2 thru_hole oval (at 0 2.54 90) (size 2.4 1.6) (drill 0.8) (layers *.Cu *.Mask) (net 45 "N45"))
  (pad 6 thru_hole oval (at 7.62 5.08 90) (size 2.4 1.6) (drill 0.8) (layers *.Cu *.Mask) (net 3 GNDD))
  (pad 3 thru_hole oval (at 0 5.08 90) (size 2.4 1.6) (drill 0.8) (layers *.Cu *.Mask) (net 31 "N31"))
  (pad 7 thru_hole oval (at 7.62 2.54 90) (size 2.4 1.6) (drill 0.8) (layers *.Cu *.Mask) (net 48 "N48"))
  (pad 4 thru_hole oval (at 0 7.62 90) (size 2.4 1.6) (drill 0.8) (layers *.Cu *.Mask) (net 3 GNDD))
  (pad 8 thru_hole oval (at 7.62 0 90) (size 2.4 1.6) (drill 0.8) (layers *.Cu *.Mask) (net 2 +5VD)))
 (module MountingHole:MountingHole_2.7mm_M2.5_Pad (layer F.Cu) (at 82.55 55.245)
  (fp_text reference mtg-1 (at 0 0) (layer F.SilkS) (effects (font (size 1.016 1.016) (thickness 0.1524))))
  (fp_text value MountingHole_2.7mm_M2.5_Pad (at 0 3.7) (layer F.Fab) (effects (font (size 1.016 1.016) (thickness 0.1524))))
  (pad 1 thru_hole circle (at 0 0) (size 5.4 5.4) (drill 2.7) (layers *.Cu *.Mask)))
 (gr_line (start 207.01 107.315) (end 207.01 50.8) (layer Edge.Cuts) (width 0.15))
 (gr_line (start 74.295 107.315) (end 207.01 107.315) (layer Edge.Cuts) (width 0.15))
 (gr_line (start 74.295 50.8) (end 74.295 107.315) (layer Edge.Cuts) (width 0.15))
 (gr_line (start 207.01 50.8) (end 74.295 50.8) (layer Edge.Cuts) (width 0.15))
 (segment (start 187.325 86.995) (end 187.325 90.17) (width 0.254) (layer F.Cu) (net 2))
 (segment (start 168.95 55.7041) (end 168.4909 55.245) (width 0.254) (layer F.Cu) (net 2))
 (segment (start 168.95 61.595) (end 168.95 55.7041) (width 0.254) (layer F.Cu) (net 2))
 (segment (start 111.085 63.54) (end 111.125 63.5) (width 0.254) (layer F.Cu) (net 2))
 (segment (start 111.085 66.675) (end 111.085 63.54) (width 0.254) (layer F.Cu) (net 2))
 (segment (start 190.624999 87.794999) (end 189.825 86.995) (width 0.254) (layer F.Cu) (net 3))
 (segment (start 192.405 89.575) (end 190.624999 87.794999) (width 0.254) (layer F.Cu) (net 3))
 (segment (start 192.405 90.17) (end 192.405 89.575) (width 0.254) (layer F.Cu) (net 3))
 (segment (start 193.459 91.624) (end 192.405 90.57) (width 0.254) (layer F.Cu) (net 3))
 (segment (start 193.859 91.624) (end 193.459 91.624) (width 0.254) (layer F.Cu) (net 3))
 (segment (start 192.405 90.57) (end 192.405 90.17) (width 0.254) (layer F.Cu) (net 3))
 (segment (start 194.945 92.71) (end 193.859 91.624) (width 0.254) (layer F.Cu) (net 3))
 (segment (start 194.945 97.79) (end 194.945 92.71) (width 0.254) (layer F.Cu) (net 3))
 (segment (start 171.0309 61.1759) (end 171.45 61.595) (width 0.254) (layer F.Cu) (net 3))
 (segment (start 171.0309 55.245) (end 171.0309 61.1759) (width 0.254) (layer F.Cu) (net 3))
 (segment (start 123.825 92.035) (end 127 88.86) (width 0.254) (layer F.Cu) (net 3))
 (segment (start 121.92 101.52) (end 123.825 99.615) (width 0.254) (layer F.Cu) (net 3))
 (segment (start 123.825 99.615) (end 123.825 92.035) (width 0.254) (layer F.Cu) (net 3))
 (segment (start 121.69 101.75) (end 121.92 101.52) (width 0.254) (layer F.Cu) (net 3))
 (segment (start 102.235 101.75) (end 121.69 101.75) (width 0.254) (layer F.Cu) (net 3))
 (segment (start 106.045 64.135) (end 106.045 63.5) (width 0.254) (layer F.Cu) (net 3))
 (segment (start 108.585 66.675) (end 106.045 64.135) (width 0.254) (layer F.Cu) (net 3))
 (segment (start 130.683 92.543) (end 127 88.86) (width 0.254) (layer F.Cu) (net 3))
 (segment (start 130.683 104.648) (end 130.683 92.543) (width 0.254) (layer F.Cu) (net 3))
 (segment (start 121.92 91.44) (end 121.92 96.52) (width 0.508) (layer F.Cu) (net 1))
 (segment (start 127 86.36) (end 121.92 91.44) (width 0.508) (layer F.Cu) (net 1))
 (segment (start 120.65 97.79) (end 121.92 96.52) (width 0.508) (layer F.Cu) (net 1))
 (segment (start 102.235 97.79) (end 120.65 97.79) (width 0.508) (layer F.Cu) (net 1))
 (segment (start 130.175 86.36) (end 130.683 85.852) (width 0.508) (layer F.Cu) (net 1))
 (segment (start 127 86.36) (end 130.175 86.36) (width 0.508) (layer F.Cu) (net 1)))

